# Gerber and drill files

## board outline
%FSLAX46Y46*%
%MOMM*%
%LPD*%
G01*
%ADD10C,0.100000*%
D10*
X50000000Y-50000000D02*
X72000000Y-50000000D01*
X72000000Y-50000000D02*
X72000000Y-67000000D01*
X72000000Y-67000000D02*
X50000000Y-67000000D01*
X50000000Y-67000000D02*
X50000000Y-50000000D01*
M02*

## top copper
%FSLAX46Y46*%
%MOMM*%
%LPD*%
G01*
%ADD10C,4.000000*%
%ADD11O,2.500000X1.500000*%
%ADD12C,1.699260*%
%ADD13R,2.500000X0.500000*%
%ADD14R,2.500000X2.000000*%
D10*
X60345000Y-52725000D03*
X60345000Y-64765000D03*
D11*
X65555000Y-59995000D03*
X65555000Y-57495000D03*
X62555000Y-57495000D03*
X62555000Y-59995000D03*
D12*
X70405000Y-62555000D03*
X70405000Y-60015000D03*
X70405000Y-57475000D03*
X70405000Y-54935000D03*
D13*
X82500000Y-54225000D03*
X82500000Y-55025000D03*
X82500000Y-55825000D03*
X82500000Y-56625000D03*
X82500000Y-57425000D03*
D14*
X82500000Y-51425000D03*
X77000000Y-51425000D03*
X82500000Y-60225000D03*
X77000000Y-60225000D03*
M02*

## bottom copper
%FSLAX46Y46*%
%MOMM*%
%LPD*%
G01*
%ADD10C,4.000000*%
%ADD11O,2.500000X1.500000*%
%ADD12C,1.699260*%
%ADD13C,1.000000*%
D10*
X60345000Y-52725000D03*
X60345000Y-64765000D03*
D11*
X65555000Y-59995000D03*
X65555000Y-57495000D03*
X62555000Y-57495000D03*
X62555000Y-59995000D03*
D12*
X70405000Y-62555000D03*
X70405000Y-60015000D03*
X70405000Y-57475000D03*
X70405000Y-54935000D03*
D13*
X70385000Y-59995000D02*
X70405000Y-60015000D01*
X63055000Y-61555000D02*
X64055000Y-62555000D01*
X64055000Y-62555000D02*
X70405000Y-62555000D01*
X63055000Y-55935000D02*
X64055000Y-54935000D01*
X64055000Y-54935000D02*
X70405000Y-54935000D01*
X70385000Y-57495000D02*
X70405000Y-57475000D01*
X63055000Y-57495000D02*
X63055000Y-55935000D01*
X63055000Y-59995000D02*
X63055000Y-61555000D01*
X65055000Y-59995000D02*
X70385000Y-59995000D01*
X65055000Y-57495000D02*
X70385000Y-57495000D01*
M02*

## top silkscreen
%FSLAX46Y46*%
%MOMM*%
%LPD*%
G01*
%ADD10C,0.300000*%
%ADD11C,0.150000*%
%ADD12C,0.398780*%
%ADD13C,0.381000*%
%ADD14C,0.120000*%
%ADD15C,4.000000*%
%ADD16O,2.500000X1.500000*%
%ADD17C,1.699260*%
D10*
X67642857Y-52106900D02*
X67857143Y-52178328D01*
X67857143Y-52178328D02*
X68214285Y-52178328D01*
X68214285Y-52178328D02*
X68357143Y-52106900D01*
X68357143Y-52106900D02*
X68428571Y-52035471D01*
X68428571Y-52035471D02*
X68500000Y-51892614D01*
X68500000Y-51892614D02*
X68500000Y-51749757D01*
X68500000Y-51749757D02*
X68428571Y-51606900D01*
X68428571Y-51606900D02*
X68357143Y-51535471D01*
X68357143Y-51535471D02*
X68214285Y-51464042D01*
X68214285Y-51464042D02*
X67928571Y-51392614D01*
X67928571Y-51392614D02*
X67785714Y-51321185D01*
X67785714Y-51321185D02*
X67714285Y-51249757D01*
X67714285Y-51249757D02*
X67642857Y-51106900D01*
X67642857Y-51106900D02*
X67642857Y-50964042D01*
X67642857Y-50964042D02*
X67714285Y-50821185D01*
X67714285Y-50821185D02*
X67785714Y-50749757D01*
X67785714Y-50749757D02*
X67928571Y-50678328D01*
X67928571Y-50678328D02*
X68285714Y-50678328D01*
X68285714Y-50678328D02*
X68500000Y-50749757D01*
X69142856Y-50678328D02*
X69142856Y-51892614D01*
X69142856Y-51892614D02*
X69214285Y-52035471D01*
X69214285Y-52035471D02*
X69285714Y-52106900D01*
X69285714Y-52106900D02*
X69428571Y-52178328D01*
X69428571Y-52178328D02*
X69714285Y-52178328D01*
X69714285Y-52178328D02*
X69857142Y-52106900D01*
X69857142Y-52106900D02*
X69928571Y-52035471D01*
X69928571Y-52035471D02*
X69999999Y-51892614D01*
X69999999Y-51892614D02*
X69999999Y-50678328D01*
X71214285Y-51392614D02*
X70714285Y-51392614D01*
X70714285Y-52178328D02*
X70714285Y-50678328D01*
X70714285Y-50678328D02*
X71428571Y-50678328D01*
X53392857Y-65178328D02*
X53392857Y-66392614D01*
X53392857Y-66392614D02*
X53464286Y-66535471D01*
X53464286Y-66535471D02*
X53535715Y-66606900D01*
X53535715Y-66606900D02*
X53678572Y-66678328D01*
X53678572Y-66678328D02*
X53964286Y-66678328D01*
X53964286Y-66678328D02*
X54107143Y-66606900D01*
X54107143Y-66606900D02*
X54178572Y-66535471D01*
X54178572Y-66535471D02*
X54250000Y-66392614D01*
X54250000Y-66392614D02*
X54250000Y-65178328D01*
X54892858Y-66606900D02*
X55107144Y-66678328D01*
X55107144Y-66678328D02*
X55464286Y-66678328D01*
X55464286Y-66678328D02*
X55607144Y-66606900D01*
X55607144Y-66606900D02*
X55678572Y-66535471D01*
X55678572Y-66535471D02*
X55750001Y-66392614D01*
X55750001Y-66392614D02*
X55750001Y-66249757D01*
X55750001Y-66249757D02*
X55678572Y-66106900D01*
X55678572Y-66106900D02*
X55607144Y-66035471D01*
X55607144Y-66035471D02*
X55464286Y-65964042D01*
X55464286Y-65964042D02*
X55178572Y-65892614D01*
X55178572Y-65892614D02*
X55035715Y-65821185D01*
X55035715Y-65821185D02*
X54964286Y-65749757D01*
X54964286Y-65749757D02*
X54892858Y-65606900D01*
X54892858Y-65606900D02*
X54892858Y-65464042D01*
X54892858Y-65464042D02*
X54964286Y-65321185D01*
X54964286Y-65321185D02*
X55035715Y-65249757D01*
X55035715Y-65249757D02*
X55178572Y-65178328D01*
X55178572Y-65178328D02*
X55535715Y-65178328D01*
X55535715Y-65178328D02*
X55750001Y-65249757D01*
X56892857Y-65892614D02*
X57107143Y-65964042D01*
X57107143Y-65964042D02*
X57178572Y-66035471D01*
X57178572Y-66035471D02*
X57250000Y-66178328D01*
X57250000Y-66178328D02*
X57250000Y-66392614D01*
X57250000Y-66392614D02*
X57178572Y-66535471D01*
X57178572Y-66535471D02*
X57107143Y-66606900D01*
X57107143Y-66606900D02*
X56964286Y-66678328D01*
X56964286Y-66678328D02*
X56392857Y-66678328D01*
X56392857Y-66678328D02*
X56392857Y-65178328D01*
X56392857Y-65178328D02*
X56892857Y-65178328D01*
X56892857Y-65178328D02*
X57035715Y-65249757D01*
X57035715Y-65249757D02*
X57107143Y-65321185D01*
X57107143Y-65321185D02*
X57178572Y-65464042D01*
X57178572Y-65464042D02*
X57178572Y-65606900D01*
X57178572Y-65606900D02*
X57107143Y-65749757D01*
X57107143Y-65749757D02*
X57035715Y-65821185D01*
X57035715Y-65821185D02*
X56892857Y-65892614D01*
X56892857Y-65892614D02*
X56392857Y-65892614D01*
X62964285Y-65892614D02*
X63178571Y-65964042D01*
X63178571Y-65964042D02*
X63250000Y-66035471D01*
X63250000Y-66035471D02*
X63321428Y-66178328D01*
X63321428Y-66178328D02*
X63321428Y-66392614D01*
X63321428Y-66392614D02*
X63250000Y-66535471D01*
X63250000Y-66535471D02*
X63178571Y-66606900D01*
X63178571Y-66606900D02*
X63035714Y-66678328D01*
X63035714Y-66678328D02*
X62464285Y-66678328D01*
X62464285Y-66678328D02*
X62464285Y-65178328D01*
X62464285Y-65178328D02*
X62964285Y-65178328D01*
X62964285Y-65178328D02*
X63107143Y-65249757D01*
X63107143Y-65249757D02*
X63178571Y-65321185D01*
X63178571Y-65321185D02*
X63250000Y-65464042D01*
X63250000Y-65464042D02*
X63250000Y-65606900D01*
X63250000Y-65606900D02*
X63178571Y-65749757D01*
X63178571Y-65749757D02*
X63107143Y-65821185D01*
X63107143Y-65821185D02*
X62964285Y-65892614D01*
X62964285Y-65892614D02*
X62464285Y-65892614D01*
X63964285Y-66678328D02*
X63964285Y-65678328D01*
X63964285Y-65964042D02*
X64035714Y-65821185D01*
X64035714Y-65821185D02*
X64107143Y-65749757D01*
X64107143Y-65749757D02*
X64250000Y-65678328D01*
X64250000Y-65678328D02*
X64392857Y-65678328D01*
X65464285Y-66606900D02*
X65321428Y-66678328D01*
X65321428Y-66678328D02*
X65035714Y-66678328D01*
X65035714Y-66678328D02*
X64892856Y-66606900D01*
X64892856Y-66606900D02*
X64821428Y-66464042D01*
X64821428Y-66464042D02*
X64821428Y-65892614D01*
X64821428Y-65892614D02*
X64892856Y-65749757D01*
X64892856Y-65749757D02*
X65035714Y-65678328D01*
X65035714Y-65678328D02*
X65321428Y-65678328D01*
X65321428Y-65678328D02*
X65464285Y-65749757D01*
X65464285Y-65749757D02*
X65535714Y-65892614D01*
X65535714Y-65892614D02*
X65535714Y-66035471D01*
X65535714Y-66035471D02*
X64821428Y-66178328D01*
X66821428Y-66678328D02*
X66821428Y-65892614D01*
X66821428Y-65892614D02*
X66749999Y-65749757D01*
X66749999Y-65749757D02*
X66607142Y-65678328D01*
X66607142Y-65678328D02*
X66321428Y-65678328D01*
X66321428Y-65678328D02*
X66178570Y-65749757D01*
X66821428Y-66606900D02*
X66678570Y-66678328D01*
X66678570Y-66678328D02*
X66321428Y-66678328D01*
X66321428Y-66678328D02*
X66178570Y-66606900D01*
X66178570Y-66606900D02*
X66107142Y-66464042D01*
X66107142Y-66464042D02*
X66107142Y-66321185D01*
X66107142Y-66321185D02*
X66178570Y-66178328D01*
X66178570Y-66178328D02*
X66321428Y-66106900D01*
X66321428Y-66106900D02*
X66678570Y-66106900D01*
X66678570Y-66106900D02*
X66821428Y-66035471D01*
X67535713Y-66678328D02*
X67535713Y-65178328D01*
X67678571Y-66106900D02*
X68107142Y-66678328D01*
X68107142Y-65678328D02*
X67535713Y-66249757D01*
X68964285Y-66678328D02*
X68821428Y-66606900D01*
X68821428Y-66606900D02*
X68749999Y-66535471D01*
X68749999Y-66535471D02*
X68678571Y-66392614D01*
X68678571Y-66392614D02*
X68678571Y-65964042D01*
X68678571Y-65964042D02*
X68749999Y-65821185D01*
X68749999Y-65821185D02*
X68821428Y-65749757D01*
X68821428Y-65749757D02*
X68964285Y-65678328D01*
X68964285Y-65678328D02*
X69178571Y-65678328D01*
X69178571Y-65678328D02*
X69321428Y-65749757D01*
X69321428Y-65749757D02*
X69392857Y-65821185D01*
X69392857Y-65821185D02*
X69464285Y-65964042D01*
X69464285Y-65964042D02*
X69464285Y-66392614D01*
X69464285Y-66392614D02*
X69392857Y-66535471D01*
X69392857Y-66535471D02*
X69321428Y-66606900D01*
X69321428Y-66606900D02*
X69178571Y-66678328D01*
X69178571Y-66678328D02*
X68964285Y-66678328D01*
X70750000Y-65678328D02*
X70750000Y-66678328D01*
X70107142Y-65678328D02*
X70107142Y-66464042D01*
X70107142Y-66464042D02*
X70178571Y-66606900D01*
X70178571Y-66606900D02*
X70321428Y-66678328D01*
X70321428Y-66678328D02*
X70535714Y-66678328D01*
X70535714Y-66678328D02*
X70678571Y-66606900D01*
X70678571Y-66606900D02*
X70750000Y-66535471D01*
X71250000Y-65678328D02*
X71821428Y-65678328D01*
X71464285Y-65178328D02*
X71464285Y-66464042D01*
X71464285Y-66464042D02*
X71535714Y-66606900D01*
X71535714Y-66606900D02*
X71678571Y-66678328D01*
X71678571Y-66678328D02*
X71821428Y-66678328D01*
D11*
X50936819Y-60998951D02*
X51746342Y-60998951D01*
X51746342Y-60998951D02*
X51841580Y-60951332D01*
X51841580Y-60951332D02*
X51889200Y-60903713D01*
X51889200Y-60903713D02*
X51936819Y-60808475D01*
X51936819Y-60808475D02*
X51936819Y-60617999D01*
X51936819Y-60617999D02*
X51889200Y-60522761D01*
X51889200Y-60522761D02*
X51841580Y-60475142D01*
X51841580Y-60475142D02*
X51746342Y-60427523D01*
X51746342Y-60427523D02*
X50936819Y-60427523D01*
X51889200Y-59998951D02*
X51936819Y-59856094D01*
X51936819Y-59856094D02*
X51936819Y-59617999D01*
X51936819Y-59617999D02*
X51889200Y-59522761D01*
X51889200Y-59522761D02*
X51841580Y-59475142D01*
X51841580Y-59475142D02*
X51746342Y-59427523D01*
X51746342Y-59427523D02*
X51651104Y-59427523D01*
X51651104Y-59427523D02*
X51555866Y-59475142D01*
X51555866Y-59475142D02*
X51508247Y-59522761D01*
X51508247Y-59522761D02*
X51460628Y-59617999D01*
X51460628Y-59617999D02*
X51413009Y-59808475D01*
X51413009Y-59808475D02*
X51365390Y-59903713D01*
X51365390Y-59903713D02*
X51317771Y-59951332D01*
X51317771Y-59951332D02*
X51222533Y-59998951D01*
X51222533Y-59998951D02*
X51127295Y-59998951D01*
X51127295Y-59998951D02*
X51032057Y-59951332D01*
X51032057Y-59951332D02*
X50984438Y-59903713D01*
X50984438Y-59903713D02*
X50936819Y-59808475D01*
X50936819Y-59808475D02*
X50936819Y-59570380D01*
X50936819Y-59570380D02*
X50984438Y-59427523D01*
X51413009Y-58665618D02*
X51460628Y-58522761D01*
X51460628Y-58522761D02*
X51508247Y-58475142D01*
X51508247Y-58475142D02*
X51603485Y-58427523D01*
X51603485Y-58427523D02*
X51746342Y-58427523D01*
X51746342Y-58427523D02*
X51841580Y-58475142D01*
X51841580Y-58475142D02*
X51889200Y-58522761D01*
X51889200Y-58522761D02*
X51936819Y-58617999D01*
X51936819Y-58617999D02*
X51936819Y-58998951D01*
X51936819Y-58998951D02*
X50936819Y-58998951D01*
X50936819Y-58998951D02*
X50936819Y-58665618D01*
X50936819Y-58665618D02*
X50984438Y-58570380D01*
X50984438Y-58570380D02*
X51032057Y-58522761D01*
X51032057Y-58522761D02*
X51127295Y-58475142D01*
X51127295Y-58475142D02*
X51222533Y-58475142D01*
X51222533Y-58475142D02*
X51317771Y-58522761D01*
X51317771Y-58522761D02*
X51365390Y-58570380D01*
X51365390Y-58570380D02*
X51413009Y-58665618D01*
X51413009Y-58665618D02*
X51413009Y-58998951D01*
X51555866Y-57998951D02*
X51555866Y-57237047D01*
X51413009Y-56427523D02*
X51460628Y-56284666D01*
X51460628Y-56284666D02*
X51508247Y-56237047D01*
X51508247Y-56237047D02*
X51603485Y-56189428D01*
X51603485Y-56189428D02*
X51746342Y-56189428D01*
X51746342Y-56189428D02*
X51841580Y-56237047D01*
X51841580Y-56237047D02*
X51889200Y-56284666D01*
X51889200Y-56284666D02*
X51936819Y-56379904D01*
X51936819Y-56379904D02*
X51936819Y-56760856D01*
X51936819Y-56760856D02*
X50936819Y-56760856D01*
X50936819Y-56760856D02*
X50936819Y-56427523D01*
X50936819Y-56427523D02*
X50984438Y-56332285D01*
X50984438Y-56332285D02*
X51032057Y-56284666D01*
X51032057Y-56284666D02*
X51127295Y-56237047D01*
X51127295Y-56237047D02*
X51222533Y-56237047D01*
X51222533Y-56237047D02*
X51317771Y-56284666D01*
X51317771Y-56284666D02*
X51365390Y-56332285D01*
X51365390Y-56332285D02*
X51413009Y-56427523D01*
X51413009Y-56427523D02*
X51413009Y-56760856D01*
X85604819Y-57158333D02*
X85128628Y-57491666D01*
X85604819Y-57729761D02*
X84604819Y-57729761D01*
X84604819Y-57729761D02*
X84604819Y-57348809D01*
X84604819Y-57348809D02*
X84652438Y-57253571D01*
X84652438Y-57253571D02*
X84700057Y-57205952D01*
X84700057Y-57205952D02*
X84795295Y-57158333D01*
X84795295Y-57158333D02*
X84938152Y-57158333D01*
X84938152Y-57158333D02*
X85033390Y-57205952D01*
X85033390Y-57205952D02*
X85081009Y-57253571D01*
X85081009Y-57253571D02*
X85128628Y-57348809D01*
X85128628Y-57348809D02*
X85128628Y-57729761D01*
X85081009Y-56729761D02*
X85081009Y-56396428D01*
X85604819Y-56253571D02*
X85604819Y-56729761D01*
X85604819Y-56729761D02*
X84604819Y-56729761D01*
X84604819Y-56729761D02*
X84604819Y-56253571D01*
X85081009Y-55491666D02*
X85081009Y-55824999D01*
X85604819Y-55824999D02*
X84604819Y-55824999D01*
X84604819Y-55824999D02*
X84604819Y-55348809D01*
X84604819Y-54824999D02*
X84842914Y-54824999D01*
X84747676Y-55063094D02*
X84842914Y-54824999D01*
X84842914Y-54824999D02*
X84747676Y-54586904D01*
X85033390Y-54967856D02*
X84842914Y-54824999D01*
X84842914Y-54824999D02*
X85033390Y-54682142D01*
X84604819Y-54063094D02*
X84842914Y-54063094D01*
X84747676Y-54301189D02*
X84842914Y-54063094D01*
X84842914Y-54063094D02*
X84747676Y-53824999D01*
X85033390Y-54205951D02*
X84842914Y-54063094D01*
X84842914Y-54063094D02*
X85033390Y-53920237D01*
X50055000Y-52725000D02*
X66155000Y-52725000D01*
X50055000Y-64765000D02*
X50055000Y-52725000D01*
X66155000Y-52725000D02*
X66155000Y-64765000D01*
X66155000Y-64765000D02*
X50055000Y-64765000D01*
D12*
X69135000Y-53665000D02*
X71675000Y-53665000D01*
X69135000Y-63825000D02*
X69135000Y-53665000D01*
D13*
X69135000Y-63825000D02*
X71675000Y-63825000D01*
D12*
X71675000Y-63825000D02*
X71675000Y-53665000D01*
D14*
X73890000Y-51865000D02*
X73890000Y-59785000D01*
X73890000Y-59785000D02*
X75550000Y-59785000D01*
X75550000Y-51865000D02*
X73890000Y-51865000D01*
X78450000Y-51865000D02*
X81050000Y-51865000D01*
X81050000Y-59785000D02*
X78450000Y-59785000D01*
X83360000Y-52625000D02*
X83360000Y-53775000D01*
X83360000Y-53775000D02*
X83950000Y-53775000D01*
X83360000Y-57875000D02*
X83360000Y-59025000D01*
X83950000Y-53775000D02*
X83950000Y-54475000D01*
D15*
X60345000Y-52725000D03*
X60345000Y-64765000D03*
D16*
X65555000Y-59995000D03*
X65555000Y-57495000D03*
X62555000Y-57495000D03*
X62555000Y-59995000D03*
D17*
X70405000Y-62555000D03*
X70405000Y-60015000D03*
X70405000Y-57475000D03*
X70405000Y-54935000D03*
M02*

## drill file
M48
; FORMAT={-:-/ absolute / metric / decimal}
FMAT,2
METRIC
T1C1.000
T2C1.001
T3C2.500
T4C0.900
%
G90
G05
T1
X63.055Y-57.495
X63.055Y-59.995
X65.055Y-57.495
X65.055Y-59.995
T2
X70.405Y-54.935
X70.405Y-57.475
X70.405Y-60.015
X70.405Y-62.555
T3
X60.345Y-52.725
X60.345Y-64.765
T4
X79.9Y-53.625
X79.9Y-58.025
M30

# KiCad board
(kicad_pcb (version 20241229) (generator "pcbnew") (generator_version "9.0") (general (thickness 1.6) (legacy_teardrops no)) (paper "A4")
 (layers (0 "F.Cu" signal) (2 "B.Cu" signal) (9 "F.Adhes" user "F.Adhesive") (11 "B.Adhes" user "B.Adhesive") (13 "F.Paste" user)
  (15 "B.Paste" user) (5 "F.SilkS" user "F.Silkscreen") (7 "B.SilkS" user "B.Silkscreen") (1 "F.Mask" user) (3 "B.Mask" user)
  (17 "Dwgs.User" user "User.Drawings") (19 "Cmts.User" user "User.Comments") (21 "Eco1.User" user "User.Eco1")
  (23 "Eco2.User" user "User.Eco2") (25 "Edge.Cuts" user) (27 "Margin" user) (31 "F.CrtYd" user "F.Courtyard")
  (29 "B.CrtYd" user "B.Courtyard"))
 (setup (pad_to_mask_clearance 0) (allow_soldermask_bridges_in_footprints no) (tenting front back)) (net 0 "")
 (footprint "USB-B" (layer "F.Cu") (at 64.055 58.745 -90)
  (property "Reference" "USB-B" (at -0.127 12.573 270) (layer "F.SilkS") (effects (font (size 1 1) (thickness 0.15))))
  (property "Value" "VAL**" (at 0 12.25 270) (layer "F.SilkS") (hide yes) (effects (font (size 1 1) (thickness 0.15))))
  (fp_line (start -6.02 14) (end -6.02 -2.1) (stroke (width 0.15) (type solid)) (layer "F.SilkS"))
  (fp_line (start 6.02 14) (end -6.02 14) (stroke (width 0.15) (type solid)) (layer "F.SilkS"))
  (fp_line (start -6.02 -2.1) (end 6.02 -2.1) (stroke (width 0.15) (type solid)) (layer "F.SilkS"))
  (fp_line (start 6.02 -2.1) (end 6.02 14) (stroke (width 0.15) (type solid)) (layer "F.SilkS"))
  (pad "" thru_hole circle (at -6.02 3.71 270) (size 4 4) (drill 2.5) (layers "*.Cu" "*.Mask" "F.SilkS") (remove_unused_layers no))
  (pad "" thru_hole circle (at 6.02 3.71 270) (size 4 4) (drill 2.5) (layers "*.Cu" "*.Mask" "F.SilkS") (remove_unused_layers no))
  (pad "1" thru_hole oval (at 1.25 -1 270) (size 1.5 2.5) (drill 1 (offset 0 -0.5)) (layers "*.Cu" "*.Mask" "F.SilkS")
   (remove_unused_layers no))
  (pad "2" thru_hole oval (at -1.25 -1 270) (size 1.5 2.5) (drill 1 (offset 0 -0.5)) (layers "*.Cu" "*.Mask" "F.SilkS")
   (remove_unused_layers no))
  (pad "3" thru_hole oval (at -1.25 1 270) (size 1.5 2.5) (drill 1 (offset 0 0.5)) (layers "*.Cu" "*.Mask" "F.SilkS")
   (remove_unused_layers no))
  (pad "4" thru_hole oval (at 1.25 1 270) (size 1.5 2.5) (drill 1 (offset 0 0.5)) (layers "*.Cu" "*.Mask" "F.SilkS")
   (remove_unused_layers no)))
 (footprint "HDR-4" (layer "F.Cu") (at 70.405 58.745 90)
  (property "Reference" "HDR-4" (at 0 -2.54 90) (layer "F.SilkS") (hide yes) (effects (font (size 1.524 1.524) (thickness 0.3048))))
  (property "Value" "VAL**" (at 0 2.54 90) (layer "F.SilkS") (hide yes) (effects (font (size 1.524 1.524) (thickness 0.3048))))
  (fp_line (start 5.08 -1.27) (end 5.08 1.27) (stroke (width 0.39878) (type solid)) (layer "F.SilkS"))
  (fp_line (start -5.08 -1.27) (end 5.08 -1.27) (stroke (width 0.39878) (type solid)) (layer "F.SilkS"))
  (fp_line (start -5.08 -1.27) (end -5.08 1.27) (stroke (width 0.381) (type solid)) (layer "F.SilkS"))
  (fp_line (start -5.08 1.27) (end 5.08 1.27) (stroke (width 0.39878) (type solid)) (layer "F.SilkS"))
  (pad "1" thru_hole circle (at -3.81 0 90) (size 1.69926 1.69926) (drill 1.00076) (layers "*.Cu" "*.Mask" "F.SilkS")
   (remove_unused_layers no))
  (pad "2" thru_hole circle (at -1.27 0 90) (size 1.69926 1.69926) (drill 1.00076) (layers "*.Cu" "*.Mask" "F.SilkS")
   (remove_unused_layers no))
  (pad "3" thru_hole circle (at 1.27 0 90) (size 1.69926 1.69926) (drill 1.00076) (layers "*.Cu" "*.Mask" "F.SilkS")
   (remove_unused_layers no))
  (pad "4" thru_hole circle (at 3.81 0 90) (size 1.69926 1.69926) (drill 1.00076) (layers "*.Cu" "*.Mask" "F.SilkS")
   (remove_unused_layers no)))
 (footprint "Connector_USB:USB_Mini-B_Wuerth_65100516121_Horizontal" (layer "F.Cu") (at 79.9 55.825 -90)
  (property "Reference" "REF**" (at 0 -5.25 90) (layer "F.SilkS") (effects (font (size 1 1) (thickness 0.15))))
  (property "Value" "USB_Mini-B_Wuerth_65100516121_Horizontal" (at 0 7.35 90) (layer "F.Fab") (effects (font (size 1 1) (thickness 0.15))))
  (fp_line (start -3.96 6.01) (end 3.96 6.01) (stroke (width 0.12) (type solid)) (layer "F.SilkS"))
  (fp_line (start 3.96 6.01) (end 3.96 4.35) (stroke (width 0.12) (type solid)) (layer "F.SilkS"))
  (fp_line (start -3.96 4.35) (end -3.96 6.01) (stroke (width 0.12) (type solid)) (layer "F.SilkS"))
  (fp_line (start -3.96 1.45) (end -3.96 -1.15) (stroke (width 0.12) (type solid)) (layer "F.SilkS"))
  (fp_line (start 3.96 -1.15) (end 3.96 1.45) (stroke (width 0.12) (type solid)) (layer "F.SilkS"))
  (fp_line (start -3.2 -3.46) (end -2.05 -3.46) (stroke (width 0.12) (type solid)) (layer "F.SilkS"))
  (fp_line (start -2.05 -3.46) (end -2.05 -4.05) (stroke (width 0.12) (type solid)) (layer "F.SilkS"))
  (fp_line (start 2.05 -3.46) (end 3.2 -3.46) (stroke (width 0.12) (type solid)) (layer "F.SilkS"))
  (fp_line (start -2.05 -4.05) (end -1.35 -4.05) (stroke (width 0.12) (type solid)) (layer "F.SilkS"))
  (pad "" np_thru_hole circle (at -2.2 0 270) (size 0.9 0.9) (drill 0.9) (layers "*.Cu" "*.Mask"))
  (pad "" np_thru_hole circle (at 2.2 0 270) (size 0.9 0.9) (drill 0.9) (layers "*.Cu" "*.Mask"))
  (pad "1" smd rect (at -1.6 -2.6 270) (size 0.5 2.5) (layers "F.Cu" "F.Mask" "F.Paste"))
  (pad "2" smd rect (at -0.8 -2.6 270) (size 0.5 2.5) (layers "F.Cu" "F.Mask" "F.Paste"))
  (pad "3" smd rect (at 0 -2.6 270) (size 0.5 2.5) (layers "F.Cu" "F.Mask" "F.Paste"))
  (pad "4" smd rect (at 0.8 -2.6 270) (size 0.5 2.5) (layers "F.Cu" "F.Mask" "F.Paste"))
  (pad "5" smd rect (at 1.6 -2.6 270) (size 0.5 2.5) (layers "F.Cu" "F.Mask" "F.Paste"))
  (pad "6" smd rect (at -4.4 -2.6 270) (size 2 2.5) (layers "F.Cu" "F.Mask" "F.Paste"))
  (pad "6" smd rect (at -4.4 2.9 270) (size 2 2.5) (layers "F.Cu" "F.Mask" "F.Paste"))
  (pad "6" smd rect (at 4.4 -2.6 270) (size 2 2.5) (layers "F.Cu" "F.Mask" "F.Paste"))
  (pad "6" smd rect (at 4.4 2.9 270) (size 2 2.5) (layers "F.Cu" "F.Mask" "F.Paste")))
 (gr_line (start 50 50) (end 72 50) (stroke (width 0.1) (type solid)) (layer "Edge.Cuts"))
 (gr_line (start 72 50) (end 72 67) (stroke (width 0.1) (type solid)) (layer "Edge.Cuts"))
 (gr_line (start 72 67) (end 50 67) (stroke (width 0.1) (type solid)) (layer "Edge.Cuts"))
 (gr_line (start 50 67) (end 50 50) (stroke (width 0.1) (type solid)) (layer "Edge.Cuts"))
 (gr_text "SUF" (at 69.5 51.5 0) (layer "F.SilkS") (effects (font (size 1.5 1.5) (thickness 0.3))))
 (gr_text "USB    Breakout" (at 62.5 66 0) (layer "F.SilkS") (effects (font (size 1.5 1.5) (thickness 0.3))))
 (segment (start 70.385 59.995) (end 70.405 60.015) (width 1) (layer "B.Cu") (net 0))
 (segment (start 63.055 61.555) (end 64.055 62.555) (width 1) (layer "B.Cu") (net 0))
 (segment (start 64.055 62.555) (end 70.405 62.555) (width 1) (layer "B.Cu") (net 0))
 (segment (start 63.055 55.935) (end 64.055 54.935) (width 1) (layer "B.Cu") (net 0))
 (segment (start 64.055 54.935) (end 70.405 54.935) (width 1) (layer "B.Cu") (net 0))
 (segment (start 70.385 57.495) (end 70.405 57.475) (width 1) (layer "B.Cu") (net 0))
 (segment (start 63.055 57.495) (end 63.055 55.935) (width 1) (layer "B.Cu") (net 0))
 (segment (start 63.055 59.995) (end 63.055 61.555) (width 1) (layer "B.Cu") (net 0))
 (segment (start 65.055 59.995) (end 70.385 59.995) (width 1) (layer "B.Cu") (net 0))
 (segment (start 65.055 57.495) (end 70.385 57.495) (width 1) (layer "B.Cu") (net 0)))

